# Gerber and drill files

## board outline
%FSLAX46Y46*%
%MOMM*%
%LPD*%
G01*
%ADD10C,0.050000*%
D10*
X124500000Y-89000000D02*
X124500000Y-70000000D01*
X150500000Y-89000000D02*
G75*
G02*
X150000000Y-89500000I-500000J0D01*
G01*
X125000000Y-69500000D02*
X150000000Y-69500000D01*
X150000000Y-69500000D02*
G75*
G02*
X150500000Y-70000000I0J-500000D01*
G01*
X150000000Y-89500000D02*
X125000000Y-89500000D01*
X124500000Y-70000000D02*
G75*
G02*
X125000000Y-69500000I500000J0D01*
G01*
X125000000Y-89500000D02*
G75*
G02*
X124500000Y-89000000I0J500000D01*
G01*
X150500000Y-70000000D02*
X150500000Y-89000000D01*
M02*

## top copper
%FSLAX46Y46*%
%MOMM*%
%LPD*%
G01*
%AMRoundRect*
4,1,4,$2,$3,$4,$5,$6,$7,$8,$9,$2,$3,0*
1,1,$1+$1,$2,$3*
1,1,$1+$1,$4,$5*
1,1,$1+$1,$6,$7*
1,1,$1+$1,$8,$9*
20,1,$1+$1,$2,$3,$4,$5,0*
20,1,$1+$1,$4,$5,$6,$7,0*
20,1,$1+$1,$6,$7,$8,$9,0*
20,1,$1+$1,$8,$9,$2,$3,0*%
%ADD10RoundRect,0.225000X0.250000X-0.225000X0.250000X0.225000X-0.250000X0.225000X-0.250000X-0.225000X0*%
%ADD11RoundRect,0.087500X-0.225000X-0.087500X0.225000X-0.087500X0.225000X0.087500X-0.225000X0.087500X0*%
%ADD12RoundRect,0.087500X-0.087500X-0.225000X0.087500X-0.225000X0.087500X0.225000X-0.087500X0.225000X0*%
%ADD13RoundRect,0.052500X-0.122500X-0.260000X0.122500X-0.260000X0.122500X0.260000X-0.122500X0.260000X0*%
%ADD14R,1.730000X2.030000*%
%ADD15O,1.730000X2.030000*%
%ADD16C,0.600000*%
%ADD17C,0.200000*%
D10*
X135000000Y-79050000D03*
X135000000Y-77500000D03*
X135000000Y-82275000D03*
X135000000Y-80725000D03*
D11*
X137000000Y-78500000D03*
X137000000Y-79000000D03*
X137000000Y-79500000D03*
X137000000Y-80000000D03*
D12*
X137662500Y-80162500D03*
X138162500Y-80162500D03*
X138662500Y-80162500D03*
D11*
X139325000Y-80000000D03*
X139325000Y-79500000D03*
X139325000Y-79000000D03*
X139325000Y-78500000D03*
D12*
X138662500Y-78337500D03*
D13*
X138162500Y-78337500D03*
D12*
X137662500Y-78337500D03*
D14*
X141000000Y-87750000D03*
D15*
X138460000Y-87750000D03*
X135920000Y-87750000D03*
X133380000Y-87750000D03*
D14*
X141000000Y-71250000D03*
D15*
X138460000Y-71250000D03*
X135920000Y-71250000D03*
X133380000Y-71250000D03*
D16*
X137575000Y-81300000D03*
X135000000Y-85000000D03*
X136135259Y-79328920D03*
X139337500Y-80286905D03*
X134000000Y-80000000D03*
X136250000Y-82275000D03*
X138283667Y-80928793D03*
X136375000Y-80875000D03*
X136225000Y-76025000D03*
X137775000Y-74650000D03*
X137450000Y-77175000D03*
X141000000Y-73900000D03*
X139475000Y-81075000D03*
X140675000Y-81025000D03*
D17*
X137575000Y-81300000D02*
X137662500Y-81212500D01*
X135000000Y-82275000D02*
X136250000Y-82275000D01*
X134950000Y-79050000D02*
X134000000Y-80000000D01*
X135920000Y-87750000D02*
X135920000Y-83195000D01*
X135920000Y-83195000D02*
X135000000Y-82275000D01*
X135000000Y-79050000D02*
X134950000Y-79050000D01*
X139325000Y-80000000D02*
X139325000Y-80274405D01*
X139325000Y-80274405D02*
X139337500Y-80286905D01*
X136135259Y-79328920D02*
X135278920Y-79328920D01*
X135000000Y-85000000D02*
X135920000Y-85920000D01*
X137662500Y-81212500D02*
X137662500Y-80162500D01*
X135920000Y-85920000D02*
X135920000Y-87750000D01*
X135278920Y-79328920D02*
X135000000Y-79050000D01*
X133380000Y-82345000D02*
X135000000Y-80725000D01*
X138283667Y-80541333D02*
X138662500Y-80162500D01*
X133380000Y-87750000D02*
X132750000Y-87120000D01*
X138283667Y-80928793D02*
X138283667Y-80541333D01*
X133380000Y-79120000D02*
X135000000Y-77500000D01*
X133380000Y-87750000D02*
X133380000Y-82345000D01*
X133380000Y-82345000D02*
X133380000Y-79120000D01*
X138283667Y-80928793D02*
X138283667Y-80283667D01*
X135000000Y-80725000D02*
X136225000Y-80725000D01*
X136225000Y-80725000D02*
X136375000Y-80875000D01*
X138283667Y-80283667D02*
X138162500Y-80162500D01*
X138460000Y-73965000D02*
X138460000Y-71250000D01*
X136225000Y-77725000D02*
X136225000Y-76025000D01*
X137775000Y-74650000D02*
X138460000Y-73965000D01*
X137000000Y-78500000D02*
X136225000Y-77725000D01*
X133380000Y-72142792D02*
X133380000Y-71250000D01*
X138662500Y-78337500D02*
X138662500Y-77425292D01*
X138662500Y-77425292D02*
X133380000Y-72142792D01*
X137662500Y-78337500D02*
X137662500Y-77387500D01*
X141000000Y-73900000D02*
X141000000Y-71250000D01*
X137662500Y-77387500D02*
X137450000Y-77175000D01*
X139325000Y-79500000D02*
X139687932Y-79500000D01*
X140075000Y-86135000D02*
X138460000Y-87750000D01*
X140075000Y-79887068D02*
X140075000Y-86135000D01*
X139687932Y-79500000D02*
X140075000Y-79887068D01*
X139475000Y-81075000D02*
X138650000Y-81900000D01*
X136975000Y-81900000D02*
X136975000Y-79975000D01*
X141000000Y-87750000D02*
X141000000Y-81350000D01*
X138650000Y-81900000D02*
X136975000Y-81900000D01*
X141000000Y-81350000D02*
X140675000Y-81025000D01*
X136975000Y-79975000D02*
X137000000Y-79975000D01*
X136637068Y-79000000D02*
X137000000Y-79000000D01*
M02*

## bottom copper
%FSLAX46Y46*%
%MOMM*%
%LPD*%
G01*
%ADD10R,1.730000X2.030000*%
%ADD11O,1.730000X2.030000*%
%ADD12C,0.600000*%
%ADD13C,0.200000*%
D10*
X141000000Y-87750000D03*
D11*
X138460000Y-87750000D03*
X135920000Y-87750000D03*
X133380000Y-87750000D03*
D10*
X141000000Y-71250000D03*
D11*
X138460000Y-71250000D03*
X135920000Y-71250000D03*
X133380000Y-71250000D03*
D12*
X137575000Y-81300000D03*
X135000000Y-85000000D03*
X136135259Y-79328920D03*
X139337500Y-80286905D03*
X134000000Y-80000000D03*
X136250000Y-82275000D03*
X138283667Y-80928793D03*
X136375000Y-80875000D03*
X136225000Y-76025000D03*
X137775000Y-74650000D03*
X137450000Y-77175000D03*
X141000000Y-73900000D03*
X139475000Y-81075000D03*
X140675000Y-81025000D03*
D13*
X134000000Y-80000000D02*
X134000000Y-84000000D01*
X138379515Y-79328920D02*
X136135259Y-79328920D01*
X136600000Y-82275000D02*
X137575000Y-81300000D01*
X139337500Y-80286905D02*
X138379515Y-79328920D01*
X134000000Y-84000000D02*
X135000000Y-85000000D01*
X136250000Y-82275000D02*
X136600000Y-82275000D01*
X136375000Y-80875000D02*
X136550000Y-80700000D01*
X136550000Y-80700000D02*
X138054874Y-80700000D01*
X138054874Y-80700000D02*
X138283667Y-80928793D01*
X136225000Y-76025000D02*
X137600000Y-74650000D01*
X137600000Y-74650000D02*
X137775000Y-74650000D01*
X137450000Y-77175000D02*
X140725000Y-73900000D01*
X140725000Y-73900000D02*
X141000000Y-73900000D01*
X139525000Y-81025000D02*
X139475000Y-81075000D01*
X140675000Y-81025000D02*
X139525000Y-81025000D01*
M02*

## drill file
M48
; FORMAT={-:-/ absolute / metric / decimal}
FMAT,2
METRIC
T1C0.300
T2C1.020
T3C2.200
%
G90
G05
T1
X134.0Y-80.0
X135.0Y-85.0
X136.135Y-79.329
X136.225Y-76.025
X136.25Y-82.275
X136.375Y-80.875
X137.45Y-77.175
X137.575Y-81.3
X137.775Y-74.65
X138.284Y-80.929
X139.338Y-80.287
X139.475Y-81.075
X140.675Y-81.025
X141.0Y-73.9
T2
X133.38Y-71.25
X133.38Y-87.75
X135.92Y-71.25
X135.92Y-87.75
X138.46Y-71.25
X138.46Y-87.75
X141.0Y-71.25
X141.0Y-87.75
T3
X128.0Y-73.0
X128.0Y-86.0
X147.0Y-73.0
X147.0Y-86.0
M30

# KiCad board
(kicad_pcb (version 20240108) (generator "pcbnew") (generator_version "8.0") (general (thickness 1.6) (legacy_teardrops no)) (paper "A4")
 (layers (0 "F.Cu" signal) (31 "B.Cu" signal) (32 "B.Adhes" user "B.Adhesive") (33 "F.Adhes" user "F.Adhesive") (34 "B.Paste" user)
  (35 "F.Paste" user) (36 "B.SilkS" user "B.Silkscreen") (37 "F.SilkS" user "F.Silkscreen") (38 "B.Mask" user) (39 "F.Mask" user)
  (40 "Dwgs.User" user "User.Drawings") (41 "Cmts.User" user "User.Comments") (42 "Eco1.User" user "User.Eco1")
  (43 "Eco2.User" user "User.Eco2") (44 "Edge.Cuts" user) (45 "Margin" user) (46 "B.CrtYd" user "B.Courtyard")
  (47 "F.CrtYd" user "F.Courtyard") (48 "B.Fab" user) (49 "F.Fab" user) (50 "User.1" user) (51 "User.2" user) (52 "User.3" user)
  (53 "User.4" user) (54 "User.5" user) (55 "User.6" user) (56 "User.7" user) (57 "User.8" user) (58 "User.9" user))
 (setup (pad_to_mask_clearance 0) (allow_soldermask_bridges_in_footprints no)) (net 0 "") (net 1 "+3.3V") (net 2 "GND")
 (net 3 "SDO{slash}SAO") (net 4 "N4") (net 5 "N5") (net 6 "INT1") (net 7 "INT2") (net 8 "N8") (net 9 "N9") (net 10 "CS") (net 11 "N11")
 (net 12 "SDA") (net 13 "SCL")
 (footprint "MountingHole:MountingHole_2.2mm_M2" (layer "F.Cu") (at 128 86)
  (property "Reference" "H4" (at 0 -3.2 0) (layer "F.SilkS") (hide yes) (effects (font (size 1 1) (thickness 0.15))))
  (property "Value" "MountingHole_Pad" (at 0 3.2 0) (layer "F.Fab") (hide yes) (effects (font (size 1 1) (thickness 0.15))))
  (pad "" np_thru_hole circle (at 0 0) (size 2.2 2.2) (drill 2.2) (layers "*.Cu" "*.Mask")))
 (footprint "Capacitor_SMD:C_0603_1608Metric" (layer "F.Cu") (at 135 78.275 90)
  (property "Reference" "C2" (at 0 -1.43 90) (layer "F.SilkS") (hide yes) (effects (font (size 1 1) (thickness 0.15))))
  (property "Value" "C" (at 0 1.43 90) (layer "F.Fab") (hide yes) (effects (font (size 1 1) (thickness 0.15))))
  (pad "1" smd roundrect (at -0.775 0 90) (size 0.9 0.95) (layers "F.Cu" "F.Paste" "F.Mask") (roundrect_rratio 0.25) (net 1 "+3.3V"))
  (pad "2" smd roundrect (at 0.775 0 90) (size 0.9 0.95) (layers "F.Cu" "F.Paste" "F.Mask") (roundrect_rratio 0.25) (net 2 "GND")))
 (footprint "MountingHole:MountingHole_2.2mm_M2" (layer "F.Cu") (at 147 86)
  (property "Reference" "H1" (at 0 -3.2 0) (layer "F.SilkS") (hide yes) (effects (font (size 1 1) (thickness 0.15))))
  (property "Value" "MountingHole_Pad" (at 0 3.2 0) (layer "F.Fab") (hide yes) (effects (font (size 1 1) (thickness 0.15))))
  (pad "" np_thru_hole circle (at 0 0) (size 2.2 2.2) (drill 2.2) (layers "*.Cu" "*.Mask")))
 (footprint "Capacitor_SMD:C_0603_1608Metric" (layer "F.Cu") (at 135 81.5 90)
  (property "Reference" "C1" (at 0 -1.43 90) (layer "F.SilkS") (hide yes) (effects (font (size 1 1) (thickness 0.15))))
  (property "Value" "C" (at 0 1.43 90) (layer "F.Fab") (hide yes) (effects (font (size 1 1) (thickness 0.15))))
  (pad "1" smd roundrect (at -0.775 0 90) (size 0.9 0.95) (layers "F.Cu" "F.Paste" "F.Mask") (roundrect_rratio 0.25) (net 1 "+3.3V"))
  (pad "2" smd roundrect (at 0.775 0 90) (size 0.9 0.95) (layers "F.Cu" "F.Paste" "F.Mask") (roundrect_rratio 0.25) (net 2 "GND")))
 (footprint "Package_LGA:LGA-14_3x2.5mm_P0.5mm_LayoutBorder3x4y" (layer "F.Cu") (at 138.1625 79.25)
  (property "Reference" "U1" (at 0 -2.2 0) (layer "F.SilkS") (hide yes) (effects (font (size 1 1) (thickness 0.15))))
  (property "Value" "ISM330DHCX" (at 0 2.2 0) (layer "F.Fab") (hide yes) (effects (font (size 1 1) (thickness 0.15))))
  (pad "1" smd roundrect (at -1.1625 -0.75) (size 0.625 0.35) (layers "F.Cu" "F.Paste" "F.Mask") (roundrect_rratio 0.25)
   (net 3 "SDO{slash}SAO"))
  (pad "2" smd roundrect (at -1.1625 -0.25) (size 0.625 0.35) (layers "F.Cu" "F.Paste" "F.Mask") (roundrect_rratio 0.25) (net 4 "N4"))
  (pad "3" smd roundrect (at -1.1625 0.25) (size 0.625 0.35) (layers "F.Cu" "F.Paste" "F.Mask") (roundrect_rratio 0.25) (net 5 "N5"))
  (pad "4" smd roundrect (at -1.1625 0.75) (size 0.625 0.35) (layers "F.Cu" "F.Paste" "F.Mask") (roundrect_rratio 0.25) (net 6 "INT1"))
  (pad "5" smd roundrect (at -0.5 0.9125) (size 0.35 0.625) (layers "F.Cu" "F.Paste" "F.Mask") (roundrect_rratio 0.25) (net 1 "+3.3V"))
  (pad "6" smd roundrect (at 0 0.9125) (size 0.35 0.625) (layers "F.Cu" "F.Paste" "F.Mask") (roundrect_rratio 0.25) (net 2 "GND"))
  (pad "7" smd roundrect (at 0.5 0.9125) (size 0.35 0.625) (layers "F.Cu" "F.Paste" "F.Mask") (roundrect_rratio 0.25) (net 2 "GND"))
  (pad "8" smd roundrect (at 1.1625 0.75) (size 0.625 0.35) (layers "F.Cu" "F.Paste" "F.Mask") (roundrect_rratio 0.25) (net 1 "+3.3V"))
  (pad "9" smd roundrect (at 1.1625 0.25) (size 0.625 0.35) (layers "F.Cu" "F.Paste" "F.Mask") (roundrect_rratio 0.25) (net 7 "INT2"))
  (pad "10" smd roundrect (at 1.1625 -0.25) (size 0.625 0.35) (layers "F.Cu" "F.Paste" "F.Mask") (roundrect_rratio 0.25) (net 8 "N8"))
  (pad "11" smd roundrect (at 1.1625 -0.75) (size 0.625 0.35) (layers "F.Cu" "F.Paste" "F.Mask") (roundrect_rratio 0.25) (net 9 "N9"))
  (pad "12" smd roundrect (at 0.5 -0.9125) (size 0.35 0.625) (layers "F.Cu" "F.Paste" "F.Mask") (roundrect_rratio 0.25) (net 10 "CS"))
  (pad "13" smd roundrect (at 0 -0.9125) (size 0.35 0.625) (layers "F.Cu" "F.Paste" "F.Mask") (roundrect_rratio 0.15) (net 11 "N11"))
  (pad "14" smd roundrect (at -0.5 -0.9125) (size 0.35 0.625) (layers "F.Cu" "F.Paste" "F.Mask") (roundrect_rratio 0.25) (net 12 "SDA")))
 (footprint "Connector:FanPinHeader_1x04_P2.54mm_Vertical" (layer "F.Cu") (at 141 87.75 180)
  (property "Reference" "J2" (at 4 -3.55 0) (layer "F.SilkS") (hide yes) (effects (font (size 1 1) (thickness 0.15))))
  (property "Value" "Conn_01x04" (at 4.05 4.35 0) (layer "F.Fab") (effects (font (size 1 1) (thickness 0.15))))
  (pad "1" thru_hole rect (at 0 0 270) (size 2.03 1.73) (drill 1.02) (layers "*.Cu" "*.Mask") (remove_unused_layers no) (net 6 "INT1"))
  (pad "2" thru_hole oval (at 2.54 0 270) (size 2.03 1.73) (drill 1.02) (layers "*.Cu" "*.Mask") (remove_unused_layers no) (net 7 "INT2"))
  (pad "3" thru_hole oval (at 5.08 0 270) (size 2.03 1.73) (drill 1.02) (layers "*.Cu" "*.Mask") (remove_unused_layers no) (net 1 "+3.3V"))
  (pad "4" thru_hole oval (at 7.62 0 270) (size 2.03 1.73) (drill 1.02) (layers "*.Cu" "*.Mask") (remove_unused_layers no) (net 2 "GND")))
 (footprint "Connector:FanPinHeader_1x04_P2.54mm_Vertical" (layer "F.Cu") (at 141 71.25 180)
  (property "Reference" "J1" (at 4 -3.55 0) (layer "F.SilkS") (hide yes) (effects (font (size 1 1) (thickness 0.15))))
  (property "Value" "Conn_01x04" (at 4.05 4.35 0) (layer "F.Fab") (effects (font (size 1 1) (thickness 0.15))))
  (pad "1" thru_hole rect (at 0 0 270) (size 2.03 1.73) (drill 1.02) (layers "*.Cu" "*.Mask") (remove_unused_layers no) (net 12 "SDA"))
  (pad "2" thru_hole oval (at 2.54 0 270) (size 2.03 1.73) (drill 1.02) (layers "*.Cu" "*.Mask") (remove_unused_layers no)
   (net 3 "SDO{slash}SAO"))
  (pad "3" thru_hole oval (at 5.08 0 270) (size 2.03 1.73) (drill 1.02) (layers "*.Cu" "*.Mask") (remove_unused_layers no) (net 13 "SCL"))
  (pad "4" thru_hole oval (at 7.62 0 270) (size 2.03 1.73) (drill 1.02) (layers "*.Cu" "*.Mask") (remove_unused_layers no) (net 10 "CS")))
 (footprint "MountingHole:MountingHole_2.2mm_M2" (layer "F.Cu") (at 147 73)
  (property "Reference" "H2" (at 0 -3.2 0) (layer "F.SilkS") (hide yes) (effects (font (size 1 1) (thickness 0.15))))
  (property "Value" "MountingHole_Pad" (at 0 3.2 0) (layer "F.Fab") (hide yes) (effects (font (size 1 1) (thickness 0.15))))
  (pad "" np_thru_hole circle (at 0 0) (size 2.2 2.2) (drill 2.2) (layers "*.Cu" "*.Mask")))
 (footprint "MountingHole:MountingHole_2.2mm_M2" (layer "F.Cu") (at 128 73)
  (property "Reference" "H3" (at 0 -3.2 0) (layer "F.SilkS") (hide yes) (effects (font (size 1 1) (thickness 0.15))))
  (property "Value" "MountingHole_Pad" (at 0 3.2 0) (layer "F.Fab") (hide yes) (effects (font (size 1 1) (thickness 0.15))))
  (pad "" np_thru_hole circle (at 0 0) (size 2.2 2.2) (drill 2.2) (layers "*.Cu" "*.Mask")))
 (gr_line (start 124.5 89) (end 124.5 70) (stroke (width 0.05) (type default)) (layer "Edge.Cuts"))
 (gr_arc (start 150.5 89) (mid 150.353553 89.353553) (end 150 89.5) (stroke (width 0.05) (type default)) (layer "Edge.Cuts"))
 (gr_line (start 125 69.5) (end 150 69.5) (stroke (width 0.05) (type default)) (layer "Edge.Cuts"))
 (gr_arc (start 150 69.5) (mid 150.353553 69.646447) (end 150.5 70) (stroke (width 0.05) (type default)) (layer "Edge.Cuts"))
 (gr_line (start 150 89.5) (end 125 89.5) (stroke (width 0.05) (type default)) (layer "Edge.Cuts"))
 (gr_arc (start 124.5 70) (mid 124.646447 69.646447) (end 125 69.5) (stroke (width 0.05) (type default)) (layer "Edge.Cuts"))
 (gr_arc (start 125 89.5) (mid 124.646447 89.353553) (end 124.5 89) (stroke (width 0.05) (type default)) (layer "Edge.Cuts"))
 (gr_line (start 150.5 70) (end 150.5 89) (stroke (width 0.05) (type default)) (layer "Edge.Cuts"))
 (segment (start 137.575 81.3) (end 137.6625 81.2125) (width 0.2) (layer "F.Cu") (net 1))
 (segment (start 135 82.275) (end 136.25 82.275) (width 0.2) (layer "F.Cu") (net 1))
 (segment (start 134.95 79.05) (end 134 80) (width 0.2) (layer "F.Cu") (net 1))
 (segment (start 135.92 87.75) (end 135.92 83.195) (width 0.2) (layer "F.Cu") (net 1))
 (segment (start 135.92 83.195) (end 135 82.275) (width 0.2) (layer "F.Cu") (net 1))
 (segment (start 135 79.05) (end 134.95 79.05) (width 0.2) (layer "F.Cu") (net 1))
 (segment (start 139.325 80) (end 139.325 80.274405) (width 0.2) (layer "F.Cu") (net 1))
 (segment (start 139.325 80.274405) (end 139.3375 80.286905) (width 0.2) (layer "F.Cu") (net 1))
 (segment (start 136.135259 79.32892) (end 135.27892 79.32892) (width 0.2) (layer "F.Cu") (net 1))
 (segment (start 135 85) (end 135.92 85.92) (width 0.2) (layer "F.Cu") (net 1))
 (segment (start 137.6625 81.2125) (end 137.6625 80.1625) (width 0.2) (layer "F.Cu") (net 1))
 (segment (start 135.92 85.92) (end 135.92 87.75) (width 0.2) (layer "F.Cu") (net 1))
 (segment (start 135.27892 79.32892) (end 135 79.05) (width 0.2) (layer "F.Cu") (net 1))
 (via (at 137.575 81.3) (size 0.6) (drill 0.3) (layers "F.Cu" "B.Cu") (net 1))
 (via (at 135 85) (size 0.6) (drill 0.3) (layers "F.Cu" "B.Cu") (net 1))
 (via (at 136.135259 79.32892) (size 0.6) (drill 0.3) (layers "F.Cu" "B.Cu") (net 1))
 (via (at 139.3375 80.286905) (size 0.6) (drill 0.3) (layers "F.Cu" "B.Cu") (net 1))
 (via (at 134 80) (size 0.6) (drill 0.3) (layers "F.Cu" "B.Cu") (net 1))
 (via (at 136.25 82.275) (size 0.6) (drill 0.3) (layers "F.Cu" "B.Cu") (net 1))
 (segment (start 134 80) (end 134 84) (width 0.2) (layer "B.Cu") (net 1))
 (segment (start 138.379515 79.32892) (end 136.135259 79.32892) (width 0.2) (layer "B.Cu") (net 1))
 (segment (start 136.6 82.275) (end 137.575 81.3) (width 0.2) (layer "B.Cu") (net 1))
 (segment (start 139.3375 80.286905) (end 138.379515 79.32892) (width 0.2) (layer "B.Cu") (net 1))
 (segment (start 134 84) (end 135 85) (width 0.2) (layer "B.Cu") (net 1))
 (segment (start 136.25 82.275) (end 136.6 82.275) (width 0.2) (layer "B.Cu") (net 1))
 (segment (start 133.38 82.345) (end 135 80.725) (width 0.2) (layer "F.Cu") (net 2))
 (segment (start 138.283667 80.541333) (end 138.6625 80.1625) (width 0.2) (layer "F.Cu") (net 2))
 (segment (start 133.38 87.75) (end 132.75 87.12) (width 0.2) (layer "F.Cu") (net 2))
 (segment (start 138.283667 80.928793) (end 138.283667 80.541333) (width 0.2) (layer "F.Cu") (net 2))
 (segment (start 133.38 79.12) (end 135 77.5) (width 0.2) (layer "F.Cu") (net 2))
 (segment (start 133.38 87.75) (end 133.38 82.345) (width 0.2) (layer "F.Cu") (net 2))
 (segment (start 133.38 82.345) (end 133.38 79.12) (width 0.2) (layer "F.Cu") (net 2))
 (segment (start 138.283667 80.928793) (end 138.283667 80.283667) (width 0.2) (layer "F.Cu") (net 2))
 (segment (start 135 80.725) (end 136.225 80.725) (width 0.2) (layer "F.Cu") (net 2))
 (segment (start 136.225 80.725) (end 136.375 80.875) (width 0.2) (layer "F.Cu") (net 2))
 (segment (start 138.283667 80.283667) (end 138.1625 80.1625) (width 0.2) (layer "F.Cu") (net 2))
 (via (at 138.283667 80.928793) (size 0.6) (drill 0.3) (layers "F.Cu" "B.Cu") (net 2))
 (via (at 136.375 80.875) (size 0.6) (drill 0.3) (layers "F.Cu" "B.Cu") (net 2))
 (segment (start 136.375 80.875) (end 136.55 80.7) (width 0.2) (layer "B.Cu") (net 2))
 (segment (start 136.55 80.7) (end 138.054874 80.7) (width 0.2) (layer "B.Cu") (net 2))
 (segment (start 138.054874 80.7) (end 138.283667 80.928793) (width 0.2) (layer "B.Cu") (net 2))
 (segment (start 138.46 73.965) (end 138.46 71.25) (width 0.2) (layer "F.Cu") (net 3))
 (segment (start 136.225 77.725) (end 136.225 76.025) (width 0.2) (layer "F.Cu") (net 3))
 (segment (start 137.775 74.65) (end 138.46 73.965) (width 0.2) (layer "F.Cu") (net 3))
 (segment (start 137 78.5) (end 136.225 77.725) (width 0.2) (layer "F.Cu") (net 3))
 (via (at 136.225 76.025) (size 0.6) (drill 0.3) (layers "F.Cu" "B.Cu") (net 3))
 (via (at 137.775 74.65) (size 0.6) (drill 0.3) (layers "F.Cu" "B.Cu") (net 3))
 (segment (start 136.225 76.025) (end 137.6 74.65) (width 0.2) (layer "B.Cu") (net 3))
 (segment (start 137.6 74.65) (end 137.775 74.65) (width 0.2) (layer "B.Cu") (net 3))
 (segment (start 133.38 72.142792) (end 133.38 71.25) (width 0.2) (layer "F.Cu") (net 10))
 (segment (start 138.6625 78.3375) (end 138.6625 77.425292) (width 0.2) (layer "F.Cu") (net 10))
 (segment (start 138.6625 77.425292) (end 133.38 72.142792) (width 0.2) (layer "F.Cu") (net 10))
 (segment (start 137.6625 78.3375) (end 137.6625 77.3875) (width 0.2) (layer "F.Cu") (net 12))
 (segment (start 141 73.9) (end 141 71.25) (width 0.2) (layer "F.Cu") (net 12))
 (segment (start 137.6625 77.3875) (end 137.45 77.175) (width 0.2) (layer "F.Cu") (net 12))
 (via (at 137.45 77.175) (size 0.6) (drill 0.3) (layers "F.Cu" "B.Cu") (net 12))
 (via (at 141 73.9) (size 0.6) (drill 0.3) (layers "F.Cu" "B.Cu") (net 12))
 (segment (start 137.45 77.175) (end 140.725 73.9) (width 0.2) (layer "B.Cu") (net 12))
 (segment (start 140.725 73.9) (end 141 73.9) (width 0.2) (layer "B.Cu") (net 12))
 (segment (start 139.325 79.5) (end 139.687932 79.5) (width 0.2) (layer "F.Cu") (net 7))
 (segment (start 140.075 86.135) (end 138.46 87.75) (width 0.2) (layer "F.Cu") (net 7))
 (segment (start 140.075 79.887068) (end 140.075 86.135) (width 0.2) (layer "F.Cu") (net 7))
 (segment (start 139.687932 79.5) (end 140.075 79.887068) (width 0.2) (layer "F.Cu") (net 7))
 (segment (start 139.475 81.075) (end 138.65 81.9) (width 0.2) (layer "F.Cu") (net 6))
 (segment (start 136.975 81.9) (end 136.975 79.975) (width 0.2) (layer "F.Cu") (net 6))
 (segment (start 141 87.75) (end 141 81.35) (width 0.2) (layer "F.Cu") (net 6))
 (segment (start 138.65 81.9) (end 136.975 81.9) (width 0.2) (layer "F.Cu") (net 6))
 (segment (start 141 81.35) (end 140.675 81.025) (width 0.2) (layer "F.Cu") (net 6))
 (segment (start 136.975 79.975) (end 137 79.975) (width 0.2) (layer "F.Cu") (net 6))
 (via (at 139.475 81.075) (size 0.6) (drill 0.3) (layers "F.Cu" "B.Cu") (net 6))
 (via (at 140.675 81.025) (size 0.6) (drill 0.3) (layers "F.Cu" "B.Cu") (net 6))
 (segment (start 139.525 81.025) (end 139.475 81.075) (width 0.2) (layer "B.Cu") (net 6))
 (segment (start 140.675 81.025) (end 139.525 81.025) (width 0.2) (layer "B.Cu") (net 6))
 (segment (start 136.637068 79) (end 137 79) (width 0.2) (layer "F.Cu") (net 4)))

